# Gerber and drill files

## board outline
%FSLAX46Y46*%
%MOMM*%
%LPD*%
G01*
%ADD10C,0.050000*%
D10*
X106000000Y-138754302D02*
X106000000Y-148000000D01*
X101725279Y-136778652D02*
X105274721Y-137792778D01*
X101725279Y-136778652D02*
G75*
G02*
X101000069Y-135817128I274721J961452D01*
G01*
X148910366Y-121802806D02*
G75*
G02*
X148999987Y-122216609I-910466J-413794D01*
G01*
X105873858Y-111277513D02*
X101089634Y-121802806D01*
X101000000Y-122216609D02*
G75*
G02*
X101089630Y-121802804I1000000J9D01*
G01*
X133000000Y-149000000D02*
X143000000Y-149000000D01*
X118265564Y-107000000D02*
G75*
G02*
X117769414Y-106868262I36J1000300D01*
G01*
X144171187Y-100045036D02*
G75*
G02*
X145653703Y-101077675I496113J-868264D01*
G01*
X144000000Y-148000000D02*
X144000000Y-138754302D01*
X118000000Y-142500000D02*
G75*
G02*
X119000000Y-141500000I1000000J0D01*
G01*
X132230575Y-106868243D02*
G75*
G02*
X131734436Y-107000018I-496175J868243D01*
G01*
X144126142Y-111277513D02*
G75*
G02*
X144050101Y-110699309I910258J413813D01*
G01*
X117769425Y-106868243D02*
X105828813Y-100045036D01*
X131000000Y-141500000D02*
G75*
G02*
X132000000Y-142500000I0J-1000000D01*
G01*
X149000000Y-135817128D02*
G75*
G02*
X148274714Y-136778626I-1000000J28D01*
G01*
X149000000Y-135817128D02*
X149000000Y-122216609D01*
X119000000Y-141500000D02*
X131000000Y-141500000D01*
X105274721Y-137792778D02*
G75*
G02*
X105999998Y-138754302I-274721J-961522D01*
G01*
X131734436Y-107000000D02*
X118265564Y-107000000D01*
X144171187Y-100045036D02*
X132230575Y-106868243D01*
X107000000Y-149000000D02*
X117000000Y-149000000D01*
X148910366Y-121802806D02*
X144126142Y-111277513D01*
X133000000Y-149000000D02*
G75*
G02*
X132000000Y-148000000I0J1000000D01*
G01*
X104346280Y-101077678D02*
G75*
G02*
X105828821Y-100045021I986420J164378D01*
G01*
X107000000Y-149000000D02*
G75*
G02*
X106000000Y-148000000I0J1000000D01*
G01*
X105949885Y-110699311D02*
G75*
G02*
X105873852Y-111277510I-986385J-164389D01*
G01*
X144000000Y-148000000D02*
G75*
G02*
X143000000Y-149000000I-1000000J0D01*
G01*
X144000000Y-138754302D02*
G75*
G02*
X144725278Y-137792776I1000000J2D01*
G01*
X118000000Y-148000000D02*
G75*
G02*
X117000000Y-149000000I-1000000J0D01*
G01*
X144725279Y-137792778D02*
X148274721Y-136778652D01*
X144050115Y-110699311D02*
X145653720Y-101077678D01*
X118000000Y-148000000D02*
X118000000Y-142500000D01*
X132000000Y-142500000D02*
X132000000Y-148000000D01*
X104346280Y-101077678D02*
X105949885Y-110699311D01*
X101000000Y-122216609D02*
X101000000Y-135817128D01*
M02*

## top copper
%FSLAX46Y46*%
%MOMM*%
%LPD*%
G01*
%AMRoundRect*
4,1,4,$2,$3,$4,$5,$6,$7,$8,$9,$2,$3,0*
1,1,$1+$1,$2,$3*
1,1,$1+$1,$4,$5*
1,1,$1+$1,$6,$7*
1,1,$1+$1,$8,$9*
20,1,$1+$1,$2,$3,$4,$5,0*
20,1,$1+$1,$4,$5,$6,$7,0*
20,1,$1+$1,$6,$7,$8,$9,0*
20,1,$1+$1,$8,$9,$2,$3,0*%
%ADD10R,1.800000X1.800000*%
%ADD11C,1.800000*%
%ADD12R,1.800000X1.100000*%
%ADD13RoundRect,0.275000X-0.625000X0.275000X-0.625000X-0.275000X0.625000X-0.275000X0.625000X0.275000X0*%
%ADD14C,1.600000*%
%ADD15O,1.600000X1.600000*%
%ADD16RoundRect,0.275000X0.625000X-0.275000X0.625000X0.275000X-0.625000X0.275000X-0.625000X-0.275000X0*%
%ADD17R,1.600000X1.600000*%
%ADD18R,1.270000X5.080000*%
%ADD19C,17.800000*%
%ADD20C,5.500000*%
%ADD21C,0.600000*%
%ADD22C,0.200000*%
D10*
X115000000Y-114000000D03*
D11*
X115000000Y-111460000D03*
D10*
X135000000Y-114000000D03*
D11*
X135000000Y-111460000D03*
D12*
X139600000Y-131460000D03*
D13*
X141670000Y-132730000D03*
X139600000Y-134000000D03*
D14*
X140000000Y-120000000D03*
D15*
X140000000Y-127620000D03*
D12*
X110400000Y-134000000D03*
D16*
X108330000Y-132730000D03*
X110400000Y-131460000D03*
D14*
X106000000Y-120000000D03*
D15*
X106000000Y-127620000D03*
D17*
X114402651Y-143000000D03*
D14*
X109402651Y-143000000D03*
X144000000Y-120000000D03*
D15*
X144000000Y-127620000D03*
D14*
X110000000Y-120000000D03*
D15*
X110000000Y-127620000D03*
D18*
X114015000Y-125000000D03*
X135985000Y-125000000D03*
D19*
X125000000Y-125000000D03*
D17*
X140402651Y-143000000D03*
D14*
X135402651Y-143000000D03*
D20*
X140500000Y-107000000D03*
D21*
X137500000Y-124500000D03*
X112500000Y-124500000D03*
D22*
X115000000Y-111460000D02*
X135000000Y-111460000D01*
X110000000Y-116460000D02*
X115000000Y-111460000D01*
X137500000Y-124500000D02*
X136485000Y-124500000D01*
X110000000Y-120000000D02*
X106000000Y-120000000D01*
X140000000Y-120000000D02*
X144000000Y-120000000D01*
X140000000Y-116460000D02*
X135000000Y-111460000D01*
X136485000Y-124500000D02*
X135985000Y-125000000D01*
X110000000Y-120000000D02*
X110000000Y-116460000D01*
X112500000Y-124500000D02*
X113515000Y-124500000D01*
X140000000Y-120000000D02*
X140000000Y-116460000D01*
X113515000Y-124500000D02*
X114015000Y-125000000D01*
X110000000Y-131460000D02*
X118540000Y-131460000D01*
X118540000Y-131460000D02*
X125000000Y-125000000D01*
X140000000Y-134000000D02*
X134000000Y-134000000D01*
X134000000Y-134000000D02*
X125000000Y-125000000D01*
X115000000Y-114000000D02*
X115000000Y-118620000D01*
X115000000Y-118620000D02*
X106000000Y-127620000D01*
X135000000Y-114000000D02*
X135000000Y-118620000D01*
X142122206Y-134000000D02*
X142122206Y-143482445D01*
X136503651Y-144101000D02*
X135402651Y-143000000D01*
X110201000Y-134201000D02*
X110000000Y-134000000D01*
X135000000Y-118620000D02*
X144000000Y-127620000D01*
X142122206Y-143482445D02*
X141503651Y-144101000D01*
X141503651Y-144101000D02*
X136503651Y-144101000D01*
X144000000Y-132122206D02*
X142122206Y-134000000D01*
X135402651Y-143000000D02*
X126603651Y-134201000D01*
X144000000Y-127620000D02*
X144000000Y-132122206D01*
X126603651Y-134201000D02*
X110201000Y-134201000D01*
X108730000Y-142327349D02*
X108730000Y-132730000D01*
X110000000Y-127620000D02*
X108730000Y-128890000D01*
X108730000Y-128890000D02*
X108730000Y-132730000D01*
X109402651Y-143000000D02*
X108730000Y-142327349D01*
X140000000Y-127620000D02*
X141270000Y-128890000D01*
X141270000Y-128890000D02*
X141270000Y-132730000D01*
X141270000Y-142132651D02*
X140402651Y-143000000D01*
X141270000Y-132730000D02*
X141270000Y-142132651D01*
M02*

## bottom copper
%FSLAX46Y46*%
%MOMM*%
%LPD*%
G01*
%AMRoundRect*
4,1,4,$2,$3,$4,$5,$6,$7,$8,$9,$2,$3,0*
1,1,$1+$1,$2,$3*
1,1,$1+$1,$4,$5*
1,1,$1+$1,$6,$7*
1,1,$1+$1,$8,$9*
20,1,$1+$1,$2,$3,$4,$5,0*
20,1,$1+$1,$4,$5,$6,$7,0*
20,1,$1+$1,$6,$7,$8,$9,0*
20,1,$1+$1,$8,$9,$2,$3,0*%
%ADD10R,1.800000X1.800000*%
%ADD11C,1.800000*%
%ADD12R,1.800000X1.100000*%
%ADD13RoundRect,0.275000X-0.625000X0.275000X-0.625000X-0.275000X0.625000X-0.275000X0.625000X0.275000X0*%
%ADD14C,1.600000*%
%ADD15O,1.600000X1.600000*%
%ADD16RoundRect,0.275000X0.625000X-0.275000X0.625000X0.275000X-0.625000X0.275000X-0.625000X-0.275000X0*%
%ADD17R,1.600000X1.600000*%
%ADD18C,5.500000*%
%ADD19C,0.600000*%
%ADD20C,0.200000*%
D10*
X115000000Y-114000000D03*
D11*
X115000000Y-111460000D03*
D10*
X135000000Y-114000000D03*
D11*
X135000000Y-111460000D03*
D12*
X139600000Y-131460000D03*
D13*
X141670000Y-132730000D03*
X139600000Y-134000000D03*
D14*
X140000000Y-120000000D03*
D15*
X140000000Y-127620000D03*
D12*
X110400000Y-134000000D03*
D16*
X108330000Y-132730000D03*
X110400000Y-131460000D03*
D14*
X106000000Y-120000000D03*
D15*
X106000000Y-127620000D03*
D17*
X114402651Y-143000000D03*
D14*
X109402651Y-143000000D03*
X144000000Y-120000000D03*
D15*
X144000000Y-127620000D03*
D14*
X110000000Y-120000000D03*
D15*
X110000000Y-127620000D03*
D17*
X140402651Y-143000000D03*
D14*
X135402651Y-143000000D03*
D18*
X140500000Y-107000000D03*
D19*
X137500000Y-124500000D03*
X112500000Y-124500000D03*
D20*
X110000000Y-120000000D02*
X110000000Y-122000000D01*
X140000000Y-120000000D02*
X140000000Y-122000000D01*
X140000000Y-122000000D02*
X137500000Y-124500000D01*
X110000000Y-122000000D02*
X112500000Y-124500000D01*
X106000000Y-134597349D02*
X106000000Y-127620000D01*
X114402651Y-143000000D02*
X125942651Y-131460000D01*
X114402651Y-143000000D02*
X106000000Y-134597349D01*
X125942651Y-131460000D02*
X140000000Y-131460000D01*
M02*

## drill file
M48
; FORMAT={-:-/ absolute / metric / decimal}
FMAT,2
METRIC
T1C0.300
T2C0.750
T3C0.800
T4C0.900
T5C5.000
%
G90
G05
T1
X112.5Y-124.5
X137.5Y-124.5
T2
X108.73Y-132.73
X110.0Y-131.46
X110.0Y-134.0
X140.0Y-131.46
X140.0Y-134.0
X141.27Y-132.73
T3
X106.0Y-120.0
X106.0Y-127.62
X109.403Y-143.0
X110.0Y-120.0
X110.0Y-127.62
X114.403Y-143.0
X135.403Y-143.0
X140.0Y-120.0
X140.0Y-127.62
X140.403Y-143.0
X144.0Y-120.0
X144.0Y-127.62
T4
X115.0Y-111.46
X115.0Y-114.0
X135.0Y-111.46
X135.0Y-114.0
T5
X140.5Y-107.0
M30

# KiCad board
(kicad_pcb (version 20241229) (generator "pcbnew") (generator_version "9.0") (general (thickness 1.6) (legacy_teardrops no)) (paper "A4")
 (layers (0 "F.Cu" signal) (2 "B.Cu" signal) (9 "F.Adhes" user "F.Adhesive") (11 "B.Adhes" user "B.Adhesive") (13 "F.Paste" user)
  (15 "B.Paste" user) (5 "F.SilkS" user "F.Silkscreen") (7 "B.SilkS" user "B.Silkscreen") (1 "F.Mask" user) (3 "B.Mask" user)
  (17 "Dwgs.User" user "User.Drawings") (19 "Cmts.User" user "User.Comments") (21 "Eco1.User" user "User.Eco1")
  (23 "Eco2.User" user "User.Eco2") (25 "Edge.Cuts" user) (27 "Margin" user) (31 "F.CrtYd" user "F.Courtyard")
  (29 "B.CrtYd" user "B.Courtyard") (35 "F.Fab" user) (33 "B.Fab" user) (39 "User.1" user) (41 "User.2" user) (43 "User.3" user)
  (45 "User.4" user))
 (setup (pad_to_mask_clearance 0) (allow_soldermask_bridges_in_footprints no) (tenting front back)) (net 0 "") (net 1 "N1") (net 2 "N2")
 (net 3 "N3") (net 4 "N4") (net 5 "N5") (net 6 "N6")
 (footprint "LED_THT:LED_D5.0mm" (layer "F.Cu") (at 115 114 90)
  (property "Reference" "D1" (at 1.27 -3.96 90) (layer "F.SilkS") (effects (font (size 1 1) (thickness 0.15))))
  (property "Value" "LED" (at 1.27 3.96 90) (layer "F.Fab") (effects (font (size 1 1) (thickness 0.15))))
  (pad "1" thru_hole rect (at 0 0 90) (size 1.8 1.8) (drill 0.9) (layers "*.Cu" "*.Mask") (remove_unused_layers no) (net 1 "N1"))
  (pad "2" thru_hole circle (at 2.54 0 90) (size 1.8 1.8) (drill 0.9) (layers "*.Cu" "*.Mask") (remove_unused_layers no) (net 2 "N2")))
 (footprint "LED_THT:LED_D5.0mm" (layer "F.Cu") (at 135 114 90)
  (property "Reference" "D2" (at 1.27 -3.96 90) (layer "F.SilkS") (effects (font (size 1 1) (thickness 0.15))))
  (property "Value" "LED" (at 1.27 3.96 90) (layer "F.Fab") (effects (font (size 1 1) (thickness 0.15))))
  (pad "1" thru_hole rect (at 0 0 90) (size 1.8 1.8) (drill 0.9) (layers "*.Cu" "*.Mask") (remove_unused_layers no) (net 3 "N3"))
  (pad "2" thru_hole circle (at 2.54 0 90) (size 1.8 1.8) (drill 0.9) (layers "*.Cu" "*.Mask") (remove_unused_layers no) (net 2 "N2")))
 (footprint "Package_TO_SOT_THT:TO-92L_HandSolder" (layer "F.Cu") (at 140 131.46 -90)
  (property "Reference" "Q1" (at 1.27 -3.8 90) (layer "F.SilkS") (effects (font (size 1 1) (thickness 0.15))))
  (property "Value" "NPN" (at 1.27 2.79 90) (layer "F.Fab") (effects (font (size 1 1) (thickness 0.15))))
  (pad "1" thru_hole rect (at 0 0 270) (size 1.1 1.8) (drill 0.75 (offset 0 0.4)) (layers "*.Cu" "*.Mask") (remove_unused_layers no)
   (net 1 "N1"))
  (pad "2" thru_hole roundrect (at 1.27 -1.27 270) (size 1.1 1.8) (drill 0.75 (offset 0 -0.4)) (layers "*.Cu" "*.Mask")
   (remove_unused_layers no) (roundrect_rratio 0.25) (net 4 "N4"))
  (pad "3" thru_hole roundrect (at 2.54 0 270) (size 1.1 1.8) (drill 0.75 (offset 0 0.4)) (layers "*.Cu" "*.Mask") (remove_unused_layers no)
   (roundrect_rratio 0.25) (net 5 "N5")))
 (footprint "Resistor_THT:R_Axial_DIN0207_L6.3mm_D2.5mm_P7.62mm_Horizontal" (layer "F.Cu") (at 140 120 -90)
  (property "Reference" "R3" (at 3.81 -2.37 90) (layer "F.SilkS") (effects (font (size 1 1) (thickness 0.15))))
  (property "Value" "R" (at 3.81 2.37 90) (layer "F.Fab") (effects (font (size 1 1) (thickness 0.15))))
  (pad "1" thru_hole circle (at 0 0 270) (size 1.6 1.6) (drill 0.8) (layers "*.Cu" "*.Mask") (remove_unused_layers no) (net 2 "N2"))
  (pad "2" thru_hole oval (at 7.62 0 270) (size 1.6 1.6) (drill 0.8) (layers "*.Cu" "*.Mask") (remove_unused_layers no) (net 4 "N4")))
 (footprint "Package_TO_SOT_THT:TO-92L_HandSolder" (layer "F.Cu") (at 110 134 90)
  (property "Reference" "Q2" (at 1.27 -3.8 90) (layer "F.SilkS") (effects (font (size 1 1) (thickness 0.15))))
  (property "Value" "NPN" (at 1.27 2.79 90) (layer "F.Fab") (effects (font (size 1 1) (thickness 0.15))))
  (pad "1" thru_hole rect (at 0 0 90) (size 1.1 1.8) (drill 0.75 (offset 0 0.4)) (layers "*.Cu" "*.Mask") (remove_unused_layers no)
   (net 3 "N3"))
  (pad "2" thru_hole roundrect (at 1.27 -1.27 90) (size 1.1 1.8) (drill 0.75 (offset 0 -0.4)) (layers "*.Cu" "*.Mask")
   (remove_unused_layers no) (roundrect_rratio 0.25) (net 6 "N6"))
  (pad "3" thru_hole roundrect (at 2.54 0 90) (size 1.1 1.8) (drill 0.75 (offset 0 0.4)) (layers "*.Cu" "*.Mask") (remove_unused_layers no)
   (roundrect_rratio 0.25) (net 5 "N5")))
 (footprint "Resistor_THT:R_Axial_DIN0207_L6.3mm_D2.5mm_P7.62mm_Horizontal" (layer "F.Cu") (at 106 120 -90)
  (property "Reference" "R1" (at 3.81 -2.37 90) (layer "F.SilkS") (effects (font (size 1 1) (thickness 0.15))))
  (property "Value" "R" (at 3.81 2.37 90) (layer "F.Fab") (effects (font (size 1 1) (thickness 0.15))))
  (pad "1" thru_hole circle (at 0 0 270) (size 1.6 1.6) (drill 0.8) (layers "*.Cu" "*.Mask") (remove_unused_layers no) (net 2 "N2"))
  (pad "2" thru_hole oval (at 7.62 0 270) (size 1.6 1.6) (drill 0.8) (layers "*.Cu" "*.Mask") (remove_unused_layers no) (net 1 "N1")))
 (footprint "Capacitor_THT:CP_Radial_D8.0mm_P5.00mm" (layer "F.Cu") (at 114.402651 143 180)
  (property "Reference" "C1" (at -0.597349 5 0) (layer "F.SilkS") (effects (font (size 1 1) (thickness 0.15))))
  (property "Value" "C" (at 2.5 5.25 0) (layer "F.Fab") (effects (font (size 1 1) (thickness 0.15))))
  (pad "1" thru_hole rect (at 0 0 180) (size 1.6 1.6) (drill 0.8) (layers "*.Cu" "*.Mask") (remove_unused_layers no) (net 1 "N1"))
  (pad "2" thru_hole circle (at 5 0 180) (size 1.6 1.6) (drill 0.8) (layers "*.Cu" "*.Mask") (remove_unused_layers no) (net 6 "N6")))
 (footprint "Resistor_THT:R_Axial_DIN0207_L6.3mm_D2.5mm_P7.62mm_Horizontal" (layer "F.Cu") (at 144 120 -90)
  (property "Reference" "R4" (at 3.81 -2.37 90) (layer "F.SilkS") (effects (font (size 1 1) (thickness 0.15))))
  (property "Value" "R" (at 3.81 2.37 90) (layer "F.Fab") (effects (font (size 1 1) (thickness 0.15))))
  (pad "1" thru_hole circle (at 0 0 270) (size 1.6 1.6) (drill 0.8) (layers "*.Cu" "*.Mask") (remove_unused_layers no) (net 2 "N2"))
  (pad "2" thru_hole oval (at 7.62 0 270) (size 1.6 1.6) (drill 0.8) (layers "*.Cu" "*.Mask") (remove_unused_layers no) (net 3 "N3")))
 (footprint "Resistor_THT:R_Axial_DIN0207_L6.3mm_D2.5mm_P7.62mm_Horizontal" (layer "F.Cu") (at 110 120 -90)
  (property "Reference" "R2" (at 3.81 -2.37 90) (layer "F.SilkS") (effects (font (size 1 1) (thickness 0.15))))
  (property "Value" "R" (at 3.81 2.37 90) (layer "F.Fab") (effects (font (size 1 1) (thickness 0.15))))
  (pad "1" thru_hole circle (at 0 0 270) (size 1.6 1.6) (drill 0.8) (layers "*.Cu" "*.Mask") (remove_unused_layers no) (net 2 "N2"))
  (pad "2" thru_hole oval (at 7.62 0 270) (size 1.6 1.6) (drill 0.8) (layers "*.Cu" "*.Mask") (remove_unused_layers no) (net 6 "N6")))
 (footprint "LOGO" (layer "F.Cu") (at 110 107)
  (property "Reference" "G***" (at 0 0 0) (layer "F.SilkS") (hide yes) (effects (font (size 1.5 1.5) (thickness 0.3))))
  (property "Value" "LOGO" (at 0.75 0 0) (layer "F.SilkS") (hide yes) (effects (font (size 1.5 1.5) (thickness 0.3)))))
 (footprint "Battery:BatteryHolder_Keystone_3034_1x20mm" (layer "F.Cu") (at 125 125)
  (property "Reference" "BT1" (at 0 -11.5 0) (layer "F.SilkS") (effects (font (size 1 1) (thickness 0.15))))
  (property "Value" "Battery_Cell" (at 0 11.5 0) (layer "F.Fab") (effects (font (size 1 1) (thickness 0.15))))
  (pad "1" smd rect (at -10.985 0) (size 1.27 5.08) (layers "F.Cu" "F.Mask" "F.Paste") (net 2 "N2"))
  (pad "1" smd rect (at 10.985 0) (size 1.27 5.08) (layers "F.Cu" "F.Mask" "F.Paste") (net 2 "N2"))
  (pad "2" smd circle (at 0 0) (size 17.8 17.8) (layers "F.Cu" "F.Mask") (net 5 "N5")))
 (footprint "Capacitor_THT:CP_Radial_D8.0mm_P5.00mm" (layer "F.Cu") (at 140.402651 143 180)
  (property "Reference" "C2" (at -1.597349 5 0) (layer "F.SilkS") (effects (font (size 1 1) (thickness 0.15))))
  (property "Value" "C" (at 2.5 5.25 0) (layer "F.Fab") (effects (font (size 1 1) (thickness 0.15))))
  (pad "1" thru_hole rect (at 0 0 180) (size 1.6 1.6) (drill 0.8) (layers "*.Cu" "*.Mask") (remove_unused_layers no) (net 4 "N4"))
  (pad "2" thru_hole circle (at 5 0 180) (size 1.6 1.6) (drill 0.8) (layers "*.Cu" "*.Mask") (remove_unused_layers no) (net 3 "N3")))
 (gr_line (start 106 138.754302) (end 106 148) (stroke (width 0.05) (type default)) (layer "Edge.Cuts"))
 (gr_line (start 101.725279 136.778652) (end 105.274721 137.792778) (stroke (width 0.05) (type default)) (layer "Edge.Cuts"))
 (gr_arc (start 101.725279 136.778652) (mid 101.201641 136.419326) (end 101 135.817128) (stroke (width 0.05) (type default))
  (layer "Edge.Cuts"))
 (gr_arc (start 148.910366 121.802806) (mid 148.977333 122.004909) (end 149 122.216609) (stroke (width 0.05) (type default))
  (layer "Edge.Cuts"))
 (gr_line (start 105.873858 111.277513) (end 101.089634 121.802806) (stroke (width 0.05) (type default)) (layer "Edge.Cuts"))
 (gr_arc (start 101 122.216609) (mid 101.022665 122.004909) (end 101.089634 121.802806) (stroke (width 0.05) (type default))
  (layer "Edge.Cuts"))
 (gr_line (start 133 149) (end 143 149) (stroke (width 0.05) (type default)) (layer "Edge.Cuts"))
 (gr_arc (start 118.265564 107) (mid 118.0089 106.966491) (end 117.769425 106.868243) (stroke (width 0.05) (type default))
  (layer "Edge.Cuts"))
 (gr_arc (start 144.171187 100.045036) (mid 145.238861 100.092734) (end 145.65372 101.077678) (stroke (width 0.05) (type default))
  (layer "Edge.Cuts"))
 (gr_line (start 144 148) (end 144 138.754302) (stroke (width 0.05) (type default)) (layer "Edge.Cuts"))
 (gr_arc (start 118 142.5) (mid 118.292893 141.792893) (end 119 141.5) (stroke (width 0.05) (type default)) (layer "Edge.Cuts"))
 (gr_arc (start 132.230575 106.868243) (mid 131.991104 106.9665) (end 131.734436 107) (stroke (width 0.05) (type default))
  (layer "Edge.Cuts"))
 (gr_arc (start 144.126142 111.277513) (mid 144.045039 110.994077) (end 144.050115 110.699311) (stroke (width 0.05) (type default))
  (layer "Edge.Cuts"))
 (gr_line (start 117.769425 106.868243) (end 105.828813 100.045036) (stroke (width 0.05) (type default)) (layer "Edge.Cuts"))
 (gr_arc (start 131 141.5) (mid 131.707107 141.792893) (end 132 142.5) (stroke (width 0.05) (type default)) (layer "Edge.Cuts"))
 (gr_arc (start 149 135.817128) (mid 148.798349 136.419324) (end 148.274721 136.778652) (stroke (width 0.05) (type default))
  (layer "Edge.Cuts"))
 (gr_line (start 149 135.817128) (end 149 122.216609) (stroke (width 0.05) (type default)) (layer "Edge.Cuts"))
 (gr_line (start 119 141.5) (end 131 141.5) (stroke (width 0.05) (type default)) (layer "Edge.Cuts"))
 (gr_arc (start 105.274721 137.792778) (mid 105.798349 138.152106) (end 106 138.754302) (stroke (width 0.05) (type default))
  (layer "Edge.Cuts"))
 (gr_line (start 131.734436 107) (end 118.265564 107) (stroke (width 0.05) (type default)) (layer "Edge.Cuts"))
 (gr_line (start 144.171187 100.045036) (end 132.230575 106.868243) (stroke (width 0.05) (type default)) (layer "Edge.Cuts"))
 (gr_line (start 107 149) (end 117 149) (stroke (width 0.05) (type default)) (layer "Edge.Cuts"))
 (gr_line (start 148.910366 121.802806) (end 144.126142 111.277513) (stroke (width 0.05) (type default)) (layer "Edge.Cuts"))
 (gr_arc (start 133 149) (mid 132.292893 148.707107) (end 132 148) (stroke (width 0.05) (type default)) (layer "Edge.Cuts"))
 (gr_arc (start 104.34628 101.077678) (mid 104.761129 100.09272) (end 105.828813 100.045036) (stroke (width 0.05) (type default))
  (layer "Edge.Cuts"))
 (gr_arc (start 107 149) (mid 106.292893 148.707107) (end 106 148) (stroke (width 0.05) (type default)) (layer "Edge.Cuts"))
 (gr_arc (start 105.949885 110.699311) (mid 105.954957 110.994077) (end 105.873858 111.277513) (stroke (width 0.05) (type default))
  (layer "Edge.Cuts"))
 (gr_arc (start 144 148) (mid 143.707107 148.707107) (end 143 149) (stroke (width 0.05) (type default)) (layer "Edge.Cuts"))
 (gr_arc (start 144 138.754302) (mid 144.201651 138.152106) (end 144.725279 137.792778) (stroke (width 0.05) (type default))
  (layer "Edge.Cuts"))
 (gr_arc (start 118 148) (mid 117.707107 148.707107) (end 117 149) (stroke (width 0.05) (type default)) (layer "Edge.Cuts"))
 (gr_line (start 144.725279 137.792778) (end 148.274721 136.778652) (stroke (width 0.05) (type default)) (layer "Edge.Cuts"))
 (gr_line (start 144.050115 110.699311) (end 145.65372 101.077678) (stroke (width 0.05) (type default)) (layer "Edge.Cuts"))
 (gr_line (start 118 148) (end 118 142.5) (stroke (width 0.05) (type default)) (layer "Edge.Cuts"))
 (gr_line (start 132 142.5) (end 132 148) (stroke (width 0.05) (type default)) (layer "Edge.Cuts"))
 (gr_line (start 104.34628 101.077678) (end 105.949885 110.699311) (stroke (width 0.05) (type default)) (layer "Edge.Cuts"))
 (gr_line (start 101 122.216609) (end 101 135.817128) (stroke (width 0.05) (type default)) (layer "Edge.Cuts"))
 (via (at 140.5 107) (size 5.5) (drill 5) (layers "F.Cu" "B.Cu") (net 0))
 (segment (start 115 111.46) (end 135 111.46) (width 0.2) (layer "F.Cu") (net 2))
 (segment (start 110 116.46) (end 115 111.46) (width 0.2) (layer "F.Cu") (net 2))
 (segment (start 137.5 124.5) (end 136.485 124.5) (width 0.2) (layer "F.Cu") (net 2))
 (segment (start 110 120) (end 106 120) (width 0.2) (layer "F.Cu") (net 2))
 (segment (start 140 120) (end 144 120) (width 0.2) (layer "F.Cu") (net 2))
 (segment (start 140 116.46) (end 135 111.46) (width 0.2) (layer "F.Cu") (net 2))
 (segment (start 136.485 124.5) (end 135.985 125) (width 0.2) (layer "F.Cu") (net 2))
 (segment (start 110 120) (end 110 116.46) (width 0.2) (layer "F.Cu") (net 2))
 (segment (start 112.5 124.5) (end 113.515 124.5) (width 0.2) (layer "F.Cu") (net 2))
 (segment (start 140 120) (end 140 116.46) (width 0.2) (layer "F.Cu") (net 2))
 (segment (start 113.515 124.5) (end 114.015 125) (width 0.2) (layer "F.Cu") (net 2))
 (via (at 137.5 124.5) (size 0.6) (drill 0.3) (layers "F.Cu" "B.Cu") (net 2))
 (via (at 112.5 124.5) (size 0.6) (drill 0.3) (layers "F.Cu" "B.Cu") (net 2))
 (segment (start 110 120) (end 110 122) (width 0.2) (layer "B.Cu") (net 2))
 (segment (start 140 120) (end 140 122) (width 0.2) (layer "B.Cu") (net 2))
 (segment (start 140 122) (end 137.5 124.5) (width 0.2) (layer "B.Cu") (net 2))
 (segment (start 110 122) (end 112.5 124.5) (width 0.2) (layer "B.Cu") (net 2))
 (segment (start 110 131.46) (end 118.54 131.46) (width 0.2) (layer "F.Cu") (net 5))
 (segment (start 118.54 131.46) (end 125 125) (width 0.2) (layer "F.Cu") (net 5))
 (segment (start 140 134) (end 134 134) (width 0.2) (layer "F.Cu") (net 5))
 (segment (start 134 134) (end 125 125) (width 0.2) (layer "F.Cu") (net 5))
 (segment (start 115 114) (end 115 118.62) (width 0.2) (layer "F.Cu") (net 1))
 (segment (start 115 118.62) (end 106 127.62) (width 0.2) (layer "F.Cu") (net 1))
 (segment (start 106 134.597349) (end 106 127.62) (width 0.2) (layer "B.Cu") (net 1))
 (segment (start 114.402651 143) (end 125.942651 131.46) (width 0.2) (layer "B.Cu") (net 1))
 (segment (start 114.402651 143) (end 106 134.597349) (width 0.2) (layer "B.Cu") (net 1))
 (segment (start 125.942651 131.46) (end 140 131.46) (width 0.2) (layer "B.Cu") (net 1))
 (segment (start 135 114) (end 135 118.62) (width 0.2) (layer "F.Cu") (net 3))
 (segment (start 142.122206 134) (end 142.122206 143.482445) (width 0.2) (layer "F.Cu") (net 3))
 (segment (start 136.503651 144.101) (end 135.402651 143) (width 0.2) (layer "F.Cu") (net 3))
 (segment (start 110.201 134.201) (end 110 134) (width 0.2) (layer "F.Cu") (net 3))
 (segment (start 135 118.62) (end 144 127.62) (width 0.2) (layer "F.Cu") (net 3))
 (segment (start 142.122206 143.482445) (end 141.503651 144.101) (width 0.2) (layer "F.Cu") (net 3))
 (segment (start 141.503651 144.101) (end 136.503651 144.101) (width 0.2) (layer "F.Cu") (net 3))
 (segment (start 144 132.122206) (end 142.122206 134) (width 0.2) (layer "F.Cu") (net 3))
 (segment (start 135.402651 143) (end 126.603651 134.201) (width 0.2) (layer "F.Cu") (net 3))
 (segment (start 144 127.62) (end 144 132.122206) (width 0.2) (layer "F.Cu") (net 3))
 (segment (start 126.603651 134.201) (end 110.201 134.201) (width 0.2) (layer "F.Cu") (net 3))
 (segment (start 108.73 142.327349) (end 108.73 132.73) (width 0.2) (layer "F.Cu") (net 6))
 (segment (start 110 127.62) (end 108.73 128.89) (width 0.2) (layer "F.Cu") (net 6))
 (segment (start 108.73 128.89) (end 108.73 132.73) (width 0.2) (layer "F.Cu") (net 6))
 (segment (start 109.402651 143) (end 108.73 142.327349) (width 0.2) (layer "F.Cu") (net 6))
 (segment (start 140 127.62) (end 141.27 128.89) (width 0.2) (layer "F.Cu") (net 4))
 (segment (start 141.27 128.89) (end 141.27 132.73) (width 0.2) (layer "F.Cu") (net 4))
 (segment (start 141.27 142.132651) (end 140.402651 143) (width 0.2) (layer "F.Cu") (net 4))
 (segment (start 141.27 132.73) (end 141.27 142.132651) (width 0.2) (layer "F.Cu") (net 4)))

